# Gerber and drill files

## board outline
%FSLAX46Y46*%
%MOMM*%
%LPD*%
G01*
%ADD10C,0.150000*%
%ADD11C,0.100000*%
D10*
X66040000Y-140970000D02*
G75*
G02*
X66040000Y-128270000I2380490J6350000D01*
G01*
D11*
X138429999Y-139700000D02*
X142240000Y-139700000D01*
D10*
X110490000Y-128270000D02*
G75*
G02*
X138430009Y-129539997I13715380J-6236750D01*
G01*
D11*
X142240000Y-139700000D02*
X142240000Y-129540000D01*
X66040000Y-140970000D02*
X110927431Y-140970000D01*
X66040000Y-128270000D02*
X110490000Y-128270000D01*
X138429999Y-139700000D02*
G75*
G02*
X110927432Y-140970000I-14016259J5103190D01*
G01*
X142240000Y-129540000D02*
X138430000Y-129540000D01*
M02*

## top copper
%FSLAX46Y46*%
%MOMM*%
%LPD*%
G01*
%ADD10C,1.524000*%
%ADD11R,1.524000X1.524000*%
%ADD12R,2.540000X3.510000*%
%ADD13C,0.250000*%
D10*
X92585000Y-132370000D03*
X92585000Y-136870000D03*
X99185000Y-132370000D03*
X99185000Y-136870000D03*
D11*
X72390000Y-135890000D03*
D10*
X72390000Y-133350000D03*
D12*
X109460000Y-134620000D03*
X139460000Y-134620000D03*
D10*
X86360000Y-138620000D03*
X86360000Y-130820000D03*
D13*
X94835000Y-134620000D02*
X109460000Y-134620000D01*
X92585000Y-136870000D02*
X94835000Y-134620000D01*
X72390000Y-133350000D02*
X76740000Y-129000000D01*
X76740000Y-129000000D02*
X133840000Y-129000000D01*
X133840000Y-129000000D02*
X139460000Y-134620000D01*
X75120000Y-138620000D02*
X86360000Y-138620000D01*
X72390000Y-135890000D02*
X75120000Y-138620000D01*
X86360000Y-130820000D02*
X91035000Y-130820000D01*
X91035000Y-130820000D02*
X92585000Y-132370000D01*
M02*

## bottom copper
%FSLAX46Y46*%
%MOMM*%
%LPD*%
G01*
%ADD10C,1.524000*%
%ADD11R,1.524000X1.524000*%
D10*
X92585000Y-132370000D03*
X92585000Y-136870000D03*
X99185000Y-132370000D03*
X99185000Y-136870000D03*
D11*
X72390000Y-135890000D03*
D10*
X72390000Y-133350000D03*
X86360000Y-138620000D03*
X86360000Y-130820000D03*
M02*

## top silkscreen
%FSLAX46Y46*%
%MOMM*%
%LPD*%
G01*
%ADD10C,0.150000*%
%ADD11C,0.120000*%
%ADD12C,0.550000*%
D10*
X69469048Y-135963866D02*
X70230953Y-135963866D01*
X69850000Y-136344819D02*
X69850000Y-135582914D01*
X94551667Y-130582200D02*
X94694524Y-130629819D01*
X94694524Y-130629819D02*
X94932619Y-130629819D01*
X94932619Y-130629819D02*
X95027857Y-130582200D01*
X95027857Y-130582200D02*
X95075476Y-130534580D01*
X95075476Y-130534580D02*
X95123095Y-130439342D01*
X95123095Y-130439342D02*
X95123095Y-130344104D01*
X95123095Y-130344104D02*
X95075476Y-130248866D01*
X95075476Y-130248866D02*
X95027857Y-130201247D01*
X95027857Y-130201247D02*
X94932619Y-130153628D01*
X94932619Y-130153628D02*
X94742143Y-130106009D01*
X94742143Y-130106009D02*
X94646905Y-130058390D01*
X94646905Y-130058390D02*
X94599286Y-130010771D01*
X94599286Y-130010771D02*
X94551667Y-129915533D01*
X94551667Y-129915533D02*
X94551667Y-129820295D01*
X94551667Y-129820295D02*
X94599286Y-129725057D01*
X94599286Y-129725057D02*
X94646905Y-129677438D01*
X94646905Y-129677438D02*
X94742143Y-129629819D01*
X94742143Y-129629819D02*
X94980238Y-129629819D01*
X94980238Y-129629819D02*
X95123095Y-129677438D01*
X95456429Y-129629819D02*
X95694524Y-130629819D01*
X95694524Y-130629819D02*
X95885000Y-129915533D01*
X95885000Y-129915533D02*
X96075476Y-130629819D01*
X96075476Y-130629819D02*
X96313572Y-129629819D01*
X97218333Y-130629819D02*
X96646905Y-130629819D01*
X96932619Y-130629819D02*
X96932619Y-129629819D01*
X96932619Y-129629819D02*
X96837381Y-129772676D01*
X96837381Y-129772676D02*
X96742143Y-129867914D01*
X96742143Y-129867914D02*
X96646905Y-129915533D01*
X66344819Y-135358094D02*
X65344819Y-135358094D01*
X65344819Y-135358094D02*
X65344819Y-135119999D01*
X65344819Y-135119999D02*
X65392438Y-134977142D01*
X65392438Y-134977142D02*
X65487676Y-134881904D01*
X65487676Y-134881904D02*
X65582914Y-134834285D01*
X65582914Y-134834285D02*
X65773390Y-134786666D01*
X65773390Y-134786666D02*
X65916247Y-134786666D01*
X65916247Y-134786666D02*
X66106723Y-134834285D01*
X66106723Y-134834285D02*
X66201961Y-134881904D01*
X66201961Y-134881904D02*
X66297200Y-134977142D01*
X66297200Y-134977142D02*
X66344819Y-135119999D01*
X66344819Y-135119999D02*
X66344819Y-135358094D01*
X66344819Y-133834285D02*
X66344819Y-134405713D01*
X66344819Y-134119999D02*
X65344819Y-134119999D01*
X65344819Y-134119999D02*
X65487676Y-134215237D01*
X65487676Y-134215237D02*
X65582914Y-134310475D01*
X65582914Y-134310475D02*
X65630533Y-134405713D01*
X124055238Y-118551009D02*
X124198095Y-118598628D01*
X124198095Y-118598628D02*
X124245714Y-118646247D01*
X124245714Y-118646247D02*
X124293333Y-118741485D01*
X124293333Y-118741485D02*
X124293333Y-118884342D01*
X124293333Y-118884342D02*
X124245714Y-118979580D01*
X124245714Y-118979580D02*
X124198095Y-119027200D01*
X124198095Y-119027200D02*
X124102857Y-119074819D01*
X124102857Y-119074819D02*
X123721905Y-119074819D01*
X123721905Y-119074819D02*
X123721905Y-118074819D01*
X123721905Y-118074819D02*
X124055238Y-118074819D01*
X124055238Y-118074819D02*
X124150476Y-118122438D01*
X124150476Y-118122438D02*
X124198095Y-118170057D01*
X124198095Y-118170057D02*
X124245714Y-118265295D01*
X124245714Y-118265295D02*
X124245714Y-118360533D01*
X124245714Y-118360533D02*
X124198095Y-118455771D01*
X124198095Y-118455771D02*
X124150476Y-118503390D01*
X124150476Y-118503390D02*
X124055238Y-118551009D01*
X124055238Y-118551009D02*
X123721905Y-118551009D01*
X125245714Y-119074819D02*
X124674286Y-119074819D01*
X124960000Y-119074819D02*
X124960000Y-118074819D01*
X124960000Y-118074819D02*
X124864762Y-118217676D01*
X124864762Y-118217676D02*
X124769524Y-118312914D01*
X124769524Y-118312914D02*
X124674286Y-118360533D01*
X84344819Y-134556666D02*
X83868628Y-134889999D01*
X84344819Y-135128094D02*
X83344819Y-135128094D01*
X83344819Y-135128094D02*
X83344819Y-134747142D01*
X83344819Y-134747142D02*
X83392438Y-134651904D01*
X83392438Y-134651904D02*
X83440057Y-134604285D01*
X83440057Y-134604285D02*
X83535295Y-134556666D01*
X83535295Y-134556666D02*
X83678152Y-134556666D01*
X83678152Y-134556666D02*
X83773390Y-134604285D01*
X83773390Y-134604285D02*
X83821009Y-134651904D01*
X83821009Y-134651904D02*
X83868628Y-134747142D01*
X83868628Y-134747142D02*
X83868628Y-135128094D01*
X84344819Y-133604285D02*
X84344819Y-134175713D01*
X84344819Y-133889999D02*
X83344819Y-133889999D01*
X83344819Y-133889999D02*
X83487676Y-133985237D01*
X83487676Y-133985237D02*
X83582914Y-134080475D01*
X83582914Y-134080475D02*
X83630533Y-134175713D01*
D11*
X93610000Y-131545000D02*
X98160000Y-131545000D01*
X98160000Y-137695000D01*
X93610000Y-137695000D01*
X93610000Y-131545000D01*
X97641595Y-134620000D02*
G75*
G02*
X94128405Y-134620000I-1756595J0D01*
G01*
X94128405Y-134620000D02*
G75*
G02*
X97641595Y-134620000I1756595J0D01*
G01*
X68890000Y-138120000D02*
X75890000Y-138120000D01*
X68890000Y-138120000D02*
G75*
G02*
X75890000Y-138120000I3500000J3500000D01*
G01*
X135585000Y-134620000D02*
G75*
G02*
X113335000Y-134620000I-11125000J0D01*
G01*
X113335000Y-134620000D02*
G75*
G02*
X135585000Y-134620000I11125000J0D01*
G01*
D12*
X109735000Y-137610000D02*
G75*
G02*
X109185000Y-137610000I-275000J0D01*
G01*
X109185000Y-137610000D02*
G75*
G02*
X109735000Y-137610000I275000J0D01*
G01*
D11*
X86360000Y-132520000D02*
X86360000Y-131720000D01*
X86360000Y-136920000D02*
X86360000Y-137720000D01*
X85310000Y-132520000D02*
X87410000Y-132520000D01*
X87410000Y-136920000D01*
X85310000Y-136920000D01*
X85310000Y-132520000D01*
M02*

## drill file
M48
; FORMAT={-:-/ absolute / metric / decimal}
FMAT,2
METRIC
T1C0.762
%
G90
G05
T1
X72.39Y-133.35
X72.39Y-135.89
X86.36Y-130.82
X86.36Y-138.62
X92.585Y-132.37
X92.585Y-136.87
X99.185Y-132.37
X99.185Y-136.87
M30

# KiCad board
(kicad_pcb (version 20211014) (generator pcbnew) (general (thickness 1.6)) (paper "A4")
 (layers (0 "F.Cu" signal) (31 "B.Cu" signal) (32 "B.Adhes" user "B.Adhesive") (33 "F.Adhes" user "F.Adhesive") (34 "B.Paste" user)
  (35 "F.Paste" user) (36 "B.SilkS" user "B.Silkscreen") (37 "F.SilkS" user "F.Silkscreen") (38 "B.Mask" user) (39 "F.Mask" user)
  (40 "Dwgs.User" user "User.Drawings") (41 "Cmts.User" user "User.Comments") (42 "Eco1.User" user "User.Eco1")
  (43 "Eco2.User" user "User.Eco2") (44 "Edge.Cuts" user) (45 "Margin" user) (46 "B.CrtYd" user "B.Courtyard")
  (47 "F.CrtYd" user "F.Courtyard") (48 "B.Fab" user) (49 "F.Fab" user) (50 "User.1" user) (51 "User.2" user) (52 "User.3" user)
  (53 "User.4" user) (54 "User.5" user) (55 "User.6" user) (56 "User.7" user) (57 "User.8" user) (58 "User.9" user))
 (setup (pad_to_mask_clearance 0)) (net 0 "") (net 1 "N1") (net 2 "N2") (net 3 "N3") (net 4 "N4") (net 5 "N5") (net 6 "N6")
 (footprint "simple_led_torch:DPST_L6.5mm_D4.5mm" (layer "F.Cu") (at 95.885 134.62)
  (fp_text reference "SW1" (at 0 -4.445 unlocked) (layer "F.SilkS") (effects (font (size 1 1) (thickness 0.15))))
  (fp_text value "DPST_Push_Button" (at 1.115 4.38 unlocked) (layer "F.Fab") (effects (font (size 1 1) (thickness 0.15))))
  (fp_rect (start -2.275 -3.075) (end 2.275 3.075) (layer "F.SilkS") (width 0.12) (fill none))
  (fp_circle (center 0 0) (end 0.725 1.6) (layer "F.SilkS") (width 0.12) (fill none))
  (pad "1" thru_hole circle (at -3.3 -2.25) (size 1.524 1.524) (drill 0.762) (layers *.Cu *.Mask) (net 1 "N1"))
  (pad "2" thru_hole circle (at -3.3 2.25) (size 1.524 1.524) (drill 0.762) (layers *.Cu *.Mask) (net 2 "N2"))
  (pad "3" thru_hole circle (at 3.3 -2.25) (size 1.524 1.524) (drill 0.762) (layers *.Cu *.Mask) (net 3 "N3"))
  (pad "4" thru_hole circle (at 3.3 2.25) (size 1.524 1.524) (drill 0.762) (layers *.Cu *.Mask) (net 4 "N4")))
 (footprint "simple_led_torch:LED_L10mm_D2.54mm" (layer "F.Cu") (at 72.39 134.62 90)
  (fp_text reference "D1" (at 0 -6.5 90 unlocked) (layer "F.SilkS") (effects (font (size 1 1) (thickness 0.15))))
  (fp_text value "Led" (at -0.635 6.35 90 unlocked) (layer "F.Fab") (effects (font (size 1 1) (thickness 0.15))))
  (fp_line (start -3.5 -3.5) (end -3.5 3.5) (layer "F.SilkS") (width 0.12))
  (fp_arc (start -3.5 -3.5) (mid 4.949747 0) (end -3.5 3.5) (layer "F.SilkS") (width 0.12))
  (pad "1" thru_hole rect (at -1.27 0 90) (size 1.524 1.524) (drill 0.762) (layers *.Cu *.Mask) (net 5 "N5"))
  (pad "2" thru_hole circle (at 1.27 0 90) (size 1.524 1.524) (drill 0.762) (layers *.Cu *.Mask) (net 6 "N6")))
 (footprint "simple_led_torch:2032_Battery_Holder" (layer "F.Cu") (at 124.46 134.62)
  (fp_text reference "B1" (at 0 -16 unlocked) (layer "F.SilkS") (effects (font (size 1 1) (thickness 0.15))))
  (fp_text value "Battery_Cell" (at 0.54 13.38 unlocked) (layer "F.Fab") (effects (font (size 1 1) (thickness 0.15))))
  (fp_circle (center 0 0) (end 11.125 0) (layer "F.SilkS") (width 0.12) (fill none))
  (fp_circle (center -15 2.99) (end -14.5 2.99) (layer "F.SilkS") (width 0.1) (fill solid))
  (pad "1" smd rect (at -15 0) (size 2.54 3.51) (layers "F.Cu" "F.Paste" "F.Mask") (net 2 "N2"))
  (pad "2" smd rect (at 15 0) (size 2.54 3.51) (layers "F.Cu" "F.Paste" "F.Mask") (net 6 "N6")))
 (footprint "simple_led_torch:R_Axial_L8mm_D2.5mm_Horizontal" (layer "F.Cu") (at 86.36 138.62 90)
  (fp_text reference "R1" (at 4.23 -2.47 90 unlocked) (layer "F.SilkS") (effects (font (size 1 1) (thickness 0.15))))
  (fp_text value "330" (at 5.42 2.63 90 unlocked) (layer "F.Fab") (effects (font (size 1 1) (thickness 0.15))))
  (fp_line (start 6.1 0) (end 6.9 0) (layer "F.SilkS") (width 0.12))
  (fp_line (start 1.7 0) (end 0.9 0) (layer "F.SilkS") (width 0.12))
  (fp_rect (start 1.7 -1.05) (end 6.1 1.05) (layer "F.SilkS") (width 0.12) (fill none))
  (pad "1" thru_hole circle (at 0 0 90) (size 1.524 1.524) (drill 0.762) (layers *.Cu *.Mask) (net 5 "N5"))
  (pad "2" thru_hole circle (at 7.8 0 90) (size 1.524 1.524) (drill 0.762) (layers *.Cu *.Mask) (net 1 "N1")))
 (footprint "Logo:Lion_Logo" (layer "B.Cu") (at 125 132 180)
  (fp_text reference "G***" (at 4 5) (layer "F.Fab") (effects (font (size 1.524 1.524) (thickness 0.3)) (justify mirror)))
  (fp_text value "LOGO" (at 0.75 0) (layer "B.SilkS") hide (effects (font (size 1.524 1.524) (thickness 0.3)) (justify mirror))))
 (gr_arc (start 66.04 140.97) (mid 61.638952 134.62) (end 66.04 128.27) (layer "Edge.Cuts") (width 0.15))
 (gr_line (start 138.429999 139.7) (end 142.24 139.7) (layer "Edge.Cuts") (width 0.1))
 (gr_arc (start 110.49 128.27) (mid 124.889523 119.455486) (end 138.43 129.54) (layer "Edge.Cuts") (width 0.15))
 (gr_line (start 142.24 139.7) (end 142.24 129.54) (layer "Edge.Cuts") (width 0.1))
 (gr_line (start 66.04 140.97) (end 110.927431 140.97) (layer "Edge.Cuts") (width 0.1))
 (gr_line (start 66.04 128.27) (end 110.49 128.27) (layer "Edge.Cuts") (width 0.1))
 (gr_arc (start 138.429999 139.7) (mid 125.101807 149.4973) (end 110.927431 140.97) (layer "Edge.Cuts") (width 0.1))
 (gr_line (start 142.24 129.54) (end 138.43 129.54) (layer "Edge.Cuts") (width 0.1))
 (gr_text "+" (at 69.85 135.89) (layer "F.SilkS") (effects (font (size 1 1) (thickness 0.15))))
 (segment (start 94.835 134.62) (end 109.46 134.62) (width 0.25) (layer "F.Cu") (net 2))
 (segment (start 92.585 136.87) (end 94.835 134.62) (width 0.25) (layer "F.Cu") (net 2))
 (segment (start 72.39 133.35) (end 76.74 129) (width 0.25) (layer "F.Cu") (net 6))
 (segment (start 76.74 129) (end 133.84 129) (width 0.25) (layer "F.Cu") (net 6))
 (segment (start 133.84 129) (end 139.46 134.62) (width 0.25) (layer "F.Cu") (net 6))
 (segment (start 75.12 138.62) (end 86.36 138.62) (width 0.25) (layer "F.Cu") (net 5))
 (segment (start 72.39 135.89) (end 75.12 138.62) (width 0.25) (layer "F.Cu") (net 5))
 (segment (start 86.36 130.82) (end 91.035 130.82) (width 0.25) (layer "F.Cu") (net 1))
 (segment (start 91.035 130.82) (end 92.585 132.37) (width 0.25) (layer "F.Cu") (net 1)))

